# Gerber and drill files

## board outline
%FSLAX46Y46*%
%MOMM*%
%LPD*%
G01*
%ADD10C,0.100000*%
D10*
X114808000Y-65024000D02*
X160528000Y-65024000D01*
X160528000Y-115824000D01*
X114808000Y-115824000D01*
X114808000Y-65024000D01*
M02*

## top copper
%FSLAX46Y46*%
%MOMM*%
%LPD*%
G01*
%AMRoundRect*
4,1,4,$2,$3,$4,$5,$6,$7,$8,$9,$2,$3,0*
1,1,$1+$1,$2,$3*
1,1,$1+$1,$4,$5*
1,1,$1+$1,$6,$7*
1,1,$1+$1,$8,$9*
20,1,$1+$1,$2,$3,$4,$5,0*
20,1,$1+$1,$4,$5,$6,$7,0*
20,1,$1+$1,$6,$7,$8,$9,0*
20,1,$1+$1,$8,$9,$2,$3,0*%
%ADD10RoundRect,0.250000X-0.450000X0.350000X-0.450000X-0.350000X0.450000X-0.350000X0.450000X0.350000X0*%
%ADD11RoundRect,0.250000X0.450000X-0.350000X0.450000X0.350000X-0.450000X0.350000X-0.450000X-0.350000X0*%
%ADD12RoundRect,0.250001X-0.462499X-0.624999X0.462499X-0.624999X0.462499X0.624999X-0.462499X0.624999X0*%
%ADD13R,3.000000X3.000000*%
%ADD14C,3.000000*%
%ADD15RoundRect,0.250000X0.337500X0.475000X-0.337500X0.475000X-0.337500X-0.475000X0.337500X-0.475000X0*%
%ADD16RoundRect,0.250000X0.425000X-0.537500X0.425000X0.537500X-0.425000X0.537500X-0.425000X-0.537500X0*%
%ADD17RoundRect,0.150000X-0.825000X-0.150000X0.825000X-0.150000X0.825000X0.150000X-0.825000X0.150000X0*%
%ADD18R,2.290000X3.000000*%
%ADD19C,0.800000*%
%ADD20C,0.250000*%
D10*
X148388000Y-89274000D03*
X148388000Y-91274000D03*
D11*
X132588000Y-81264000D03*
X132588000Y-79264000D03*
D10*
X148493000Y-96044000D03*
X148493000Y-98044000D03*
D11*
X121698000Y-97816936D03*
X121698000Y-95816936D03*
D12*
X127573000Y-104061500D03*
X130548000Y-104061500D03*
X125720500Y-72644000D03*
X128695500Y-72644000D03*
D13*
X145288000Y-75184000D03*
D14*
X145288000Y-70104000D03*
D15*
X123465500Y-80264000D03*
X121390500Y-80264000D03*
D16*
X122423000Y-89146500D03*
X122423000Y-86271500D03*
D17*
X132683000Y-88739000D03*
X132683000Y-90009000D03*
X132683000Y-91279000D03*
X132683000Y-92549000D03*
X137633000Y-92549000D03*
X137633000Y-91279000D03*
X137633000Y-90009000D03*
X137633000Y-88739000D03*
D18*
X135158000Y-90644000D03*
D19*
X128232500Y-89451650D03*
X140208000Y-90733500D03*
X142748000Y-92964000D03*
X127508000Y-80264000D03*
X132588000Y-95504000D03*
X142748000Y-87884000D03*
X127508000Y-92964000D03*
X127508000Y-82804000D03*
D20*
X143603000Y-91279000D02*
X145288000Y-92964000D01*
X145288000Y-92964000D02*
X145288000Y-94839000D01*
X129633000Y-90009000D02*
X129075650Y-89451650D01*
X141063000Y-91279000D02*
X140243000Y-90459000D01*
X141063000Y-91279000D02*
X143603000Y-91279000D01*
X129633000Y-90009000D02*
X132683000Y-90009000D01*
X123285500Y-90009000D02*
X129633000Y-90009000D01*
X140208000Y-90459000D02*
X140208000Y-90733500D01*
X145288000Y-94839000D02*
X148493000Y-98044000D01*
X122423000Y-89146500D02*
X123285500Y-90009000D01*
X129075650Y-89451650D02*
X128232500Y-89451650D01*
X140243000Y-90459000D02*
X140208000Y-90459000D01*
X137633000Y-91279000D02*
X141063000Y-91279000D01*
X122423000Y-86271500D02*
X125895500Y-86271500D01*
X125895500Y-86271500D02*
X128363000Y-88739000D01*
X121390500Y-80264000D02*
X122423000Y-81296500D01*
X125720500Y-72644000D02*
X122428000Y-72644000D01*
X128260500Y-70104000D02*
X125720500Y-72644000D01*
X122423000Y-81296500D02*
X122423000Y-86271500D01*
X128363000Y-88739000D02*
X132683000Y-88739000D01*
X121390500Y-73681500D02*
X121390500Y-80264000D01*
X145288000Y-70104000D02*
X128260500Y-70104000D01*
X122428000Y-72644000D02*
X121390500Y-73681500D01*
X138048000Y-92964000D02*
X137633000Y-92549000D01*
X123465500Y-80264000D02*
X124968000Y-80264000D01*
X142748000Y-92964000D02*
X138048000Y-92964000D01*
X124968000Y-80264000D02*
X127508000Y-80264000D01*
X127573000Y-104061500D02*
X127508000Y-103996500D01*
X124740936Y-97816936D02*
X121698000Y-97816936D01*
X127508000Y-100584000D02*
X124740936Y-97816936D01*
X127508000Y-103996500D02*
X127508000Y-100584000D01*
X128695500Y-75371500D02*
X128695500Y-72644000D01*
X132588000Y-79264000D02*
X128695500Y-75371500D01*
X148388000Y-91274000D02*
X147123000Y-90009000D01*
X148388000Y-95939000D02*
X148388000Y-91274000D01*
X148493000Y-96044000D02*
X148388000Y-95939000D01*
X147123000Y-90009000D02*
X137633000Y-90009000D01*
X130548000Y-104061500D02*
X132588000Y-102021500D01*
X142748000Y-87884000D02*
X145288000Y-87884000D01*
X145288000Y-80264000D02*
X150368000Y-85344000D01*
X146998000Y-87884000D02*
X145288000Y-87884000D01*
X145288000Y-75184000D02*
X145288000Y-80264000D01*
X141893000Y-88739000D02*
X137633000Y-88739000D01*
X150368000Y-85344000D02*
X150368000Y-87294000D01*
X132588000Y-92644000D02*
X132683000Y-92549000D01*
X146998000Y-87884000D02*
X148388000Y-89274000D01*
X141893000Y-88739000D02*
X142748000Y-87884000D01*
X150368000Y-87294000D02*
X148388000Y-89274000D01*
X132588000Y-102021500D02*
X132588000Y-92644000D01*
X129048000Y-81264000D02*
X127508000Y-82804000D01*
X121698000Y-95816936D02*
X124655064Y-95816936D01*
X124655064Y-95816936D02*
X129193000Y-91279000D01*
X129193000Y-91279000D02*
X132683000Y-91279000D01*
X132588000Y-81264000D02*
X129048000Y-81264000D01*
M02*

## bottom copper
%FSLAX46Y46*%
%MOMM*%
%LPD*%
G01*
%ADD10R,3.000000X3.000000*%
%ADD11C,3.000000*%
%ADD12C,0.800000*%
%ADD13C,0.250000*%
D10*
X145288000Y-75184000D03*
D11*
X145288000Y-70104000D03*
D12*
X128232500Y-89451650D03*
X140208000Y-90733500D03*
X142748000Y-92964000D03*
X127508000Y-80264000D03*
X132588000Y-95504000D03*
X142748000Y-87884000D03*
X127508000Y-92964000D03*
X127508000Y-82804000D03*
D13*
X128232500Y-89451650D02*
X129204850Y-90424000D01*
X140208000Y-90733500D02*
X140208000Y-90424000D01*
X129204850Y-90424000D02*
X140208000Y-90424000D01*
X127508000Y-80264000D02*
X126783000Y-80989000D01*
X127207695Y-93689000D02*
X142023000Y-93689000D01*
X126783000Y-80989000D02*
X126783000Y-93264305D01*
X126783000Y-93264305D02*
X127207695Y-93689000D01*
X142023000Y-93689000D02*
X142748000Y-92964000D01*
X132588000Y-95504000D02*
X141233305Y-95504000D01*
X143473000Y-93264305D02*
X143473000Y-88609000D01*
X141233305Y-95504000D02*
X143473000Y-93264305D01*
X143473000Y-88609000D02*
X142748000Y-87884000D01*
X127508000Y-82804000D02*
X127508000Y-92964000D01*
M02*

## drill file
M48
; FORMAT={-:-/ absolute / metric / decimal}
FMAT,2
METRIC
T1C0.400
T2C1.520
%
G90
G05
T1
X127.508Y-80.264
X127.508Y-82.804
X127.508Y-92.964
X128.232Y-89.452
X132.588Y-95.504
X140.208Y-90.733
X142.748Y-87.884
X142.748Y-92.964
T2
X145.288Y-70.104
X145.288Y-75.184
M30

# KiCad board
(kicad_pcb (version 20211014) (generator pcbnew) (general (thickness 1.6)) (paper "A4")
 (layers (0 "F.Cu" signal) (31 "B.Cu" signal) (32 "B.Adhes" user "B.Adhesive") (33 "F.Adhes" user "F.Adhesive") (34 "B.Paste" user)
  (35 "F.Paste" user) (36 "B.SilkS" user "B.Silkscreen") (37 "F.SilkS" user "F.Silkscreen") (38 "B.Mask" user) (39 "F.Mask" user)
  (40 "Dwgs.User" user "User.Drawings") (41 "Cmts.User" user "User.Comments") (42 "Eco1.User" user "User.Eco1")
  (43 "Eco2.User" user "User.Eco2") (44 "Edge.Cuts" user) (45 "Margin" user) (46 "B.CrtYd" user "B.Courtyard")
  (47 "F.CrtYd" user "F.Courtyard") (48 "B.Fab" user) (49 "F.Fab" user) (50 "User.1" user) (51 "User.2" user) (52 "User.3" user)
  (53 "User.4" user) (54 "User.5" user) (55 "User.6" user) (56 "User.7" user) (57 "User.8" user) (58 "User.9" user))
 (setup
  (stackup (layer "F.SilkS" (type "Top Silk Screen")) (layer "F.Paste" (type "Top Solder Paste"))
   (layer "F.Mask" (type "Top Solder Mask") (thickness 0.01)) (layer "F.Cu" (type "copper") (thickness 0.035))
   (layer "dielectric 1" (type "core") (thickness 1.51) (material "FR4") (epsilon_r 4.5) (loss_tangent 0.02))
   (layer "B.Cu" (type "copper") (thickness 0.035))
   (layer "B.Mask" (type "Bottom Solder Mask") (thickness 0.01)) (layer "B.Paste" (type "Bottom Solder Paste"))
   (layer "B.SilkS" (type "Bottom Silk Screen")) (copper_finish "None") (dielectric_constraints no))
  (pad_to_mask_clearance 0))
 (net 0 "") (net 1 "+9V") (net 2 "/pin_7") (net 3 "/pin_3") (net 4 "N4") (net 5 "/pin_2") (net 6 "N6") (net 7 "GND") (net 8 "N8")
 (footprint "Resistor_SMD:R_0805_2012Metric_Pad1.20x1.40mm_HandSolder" (layer "F.Cu") (at 148.388 90.274 -90)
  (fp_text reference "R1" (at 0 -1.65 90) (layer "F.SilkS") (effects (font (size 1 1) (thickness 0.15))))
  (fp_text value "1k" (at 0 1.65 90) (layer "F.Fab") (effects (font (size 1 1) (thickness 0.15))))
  (pad "1" smd roundrect (at -1 0 270) (size 1.2 1.4) (layers "F.Cu" "F.Paste" "F.Mask") (roundrect_rratio 0.208333) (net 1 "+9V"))
  (pad "2" smd roundrect (at 1 0 270) (size 1.2 1.4) (layers "F.Cu" "F.Paste" "F.Mask") (roundrect_rratio 0.208333) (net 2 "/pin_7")))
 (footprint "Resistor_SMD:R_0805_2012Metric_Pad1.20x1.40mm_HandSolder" (layer "F.Cu") (at 132.588 80.264 90)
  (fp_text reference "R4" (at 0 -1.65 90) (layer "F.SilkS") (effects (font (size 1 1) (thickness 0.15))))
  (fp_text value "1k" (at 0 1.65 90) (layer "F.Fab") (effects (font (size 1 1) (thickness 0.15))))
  (pad "1" smd roundrect (at -1 0 90) (size 1.2 1.4) (layers "F.Cu" "F.Paste" "F.Mask") (roundrect_rratio 0.208333) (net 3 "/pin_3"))
  (pad "2" smd roundrect (at 1 0 90) (size 1.2 1.4) (layers "F.Cu" "F.Paste" "F.Mask") (roundrect_rratio 0.208333) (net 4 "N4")))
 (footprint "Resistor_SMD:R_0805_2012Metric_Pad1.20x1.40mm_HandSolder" (layer "F.Cu") (at 148.493 97.044 -90)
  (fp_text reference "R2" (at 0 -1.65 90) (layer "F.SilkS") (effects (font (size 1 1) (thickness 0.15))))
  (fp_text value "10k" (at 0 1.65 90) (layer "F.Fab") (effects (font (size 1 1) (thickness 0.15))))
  (pad "1" smd roundrect (at -1 0 270) (size 1.2 1.4) (layers "F.Cu" "F.Paste" "F.Mask") (roundrect_rratio 0.208333) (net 2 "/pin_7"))
  (pad "2" smd roundrect (at 1 0 270) (size 1.2 1.4) (layers "F.Cu" "F.Paste" "F.Mask") (roundrect_rratio 0.208333) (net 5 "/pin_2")))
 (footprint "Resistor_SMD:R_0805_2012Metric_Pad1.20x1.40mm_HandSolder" (layer "F.Cu") (at 121.698 96.816936 90)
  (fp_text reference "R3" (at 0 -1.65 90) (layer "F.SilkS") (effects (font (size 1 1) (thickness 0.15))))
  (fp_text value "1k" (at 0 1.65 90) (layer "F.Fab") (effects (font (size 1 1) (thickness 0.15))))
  (pad "1" smd roundrect (at -1 0 90) (size 1.2 1.4) (layers "F.Cu" "F.Paste" "F.Mask") (roundrect_rratio 0.208333) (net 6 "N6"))
  (pad "2" smd roundrect (at 1 0 90) (size 1.2 1.4) (layers "F.Cu" "F.Paste" "F.Mask") (roundrect_rratio 0.208333) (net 3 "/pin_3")))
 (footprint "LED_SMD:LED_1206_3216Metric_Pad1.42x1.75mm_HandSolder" (layer "F.Cu") (at 129.0605 104.0615)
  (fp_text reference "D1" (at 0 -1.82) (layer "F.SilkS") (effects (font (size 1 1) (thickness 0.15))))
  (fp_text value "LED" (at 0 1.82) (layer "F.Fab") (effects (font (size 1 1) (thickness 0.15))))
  (pad "1" smd roundrect (at -1.4875 0) (size 1.425 1.75) (layers "F.Cu" "F.Paste" "F.Mask") (roundrect_rratio 0.175439) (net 6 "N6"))
  (pad "2" smd roundrect (at 1.4875 0) (size 1.425 1.75) (layers "F.Cu" "F.Paste" "F.Mask") (roundrect_rratio 0.175439) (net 1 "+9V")))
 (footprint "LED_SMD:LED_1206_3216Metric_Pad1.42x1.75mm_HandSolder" (layer "F.Cu") (at 127.208 72.644)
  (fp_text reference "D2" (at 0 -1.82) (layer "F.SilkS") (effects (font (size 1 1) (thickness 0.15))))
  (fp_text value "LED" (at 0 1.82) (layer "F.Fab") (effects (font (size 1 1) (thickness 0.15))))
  (pad "1" smd roundrect (at -1.4875 0) (size 1.425 1.75) (layers "F.Cu" "F.Paste" "F.Mask") (roundrect_rratio 0.175439) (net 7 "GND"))
  (pad "2" smd roundrect (at 1.4875 0) (size 1.425 1.75) (layers "F.Cu" "F.Paste" "F.Mask") (roundrect_rratio 0.175439) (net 4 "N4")))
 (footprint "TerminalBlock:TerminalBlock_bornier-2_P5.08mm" (layer "F.Cu") (at 145.288 75.184 90)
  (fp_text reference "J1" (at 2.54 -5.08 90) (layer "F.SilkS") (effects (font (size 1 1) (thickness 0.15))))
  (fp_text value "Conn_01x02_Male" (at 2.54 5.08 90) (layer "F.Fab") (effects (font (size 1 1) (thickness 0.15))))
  (pad "1" thru_hole rect (at 0 0 90) (size 3 3) (drill 1.52) (layers F&B.Cu *.Mask) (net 1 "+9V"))
  (pad "2" thru_hole circle (at 5.08 0 90) (size 3 3) (drill 1.52) (layers F&B.Cu *.Mask) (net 7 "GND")))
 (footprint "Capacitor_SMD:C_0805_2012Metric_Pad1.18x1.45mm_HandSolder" (layer "F.Cu") (at 122.428 80.264 180)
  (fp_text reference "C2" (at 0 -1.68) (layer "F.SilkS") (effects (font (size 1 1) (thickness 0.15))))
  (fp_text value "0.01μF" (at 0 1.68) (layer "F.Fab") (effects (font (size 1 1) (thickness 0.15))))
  (pad "1" smd roundrect (at -1.0375 0 180) (size 1.175 1.45) (layers "F.Cu" "F.Paste" "F.Mask") (roundrect_rratio 0.212766) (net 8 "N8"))
  (pad "2" smd roundrect (at 1.0375 0 180) (size 1.175 1.45) (layers "F.Cu" "F.Paste" "F.Mask") (roundrect_rratio 0.212766) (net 7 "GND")))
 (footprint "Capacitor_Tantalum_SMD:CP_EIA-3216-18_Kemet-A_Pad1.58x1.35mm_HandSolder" (layer "F.Cu") (at 122.423 87.709 90)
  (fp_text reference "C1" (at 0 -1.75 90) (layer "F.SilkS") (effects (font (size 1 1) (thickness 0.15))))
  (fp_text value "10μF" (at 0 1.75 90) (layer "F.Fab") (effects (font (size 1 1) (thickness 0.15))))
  (pad "1" smd roundrect (at -1.4375 0 90) (size 1.575 1.35) (layers "F.Cu" "F.Paste" "F.Mask") (roundrect_rratio 0.185185) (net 5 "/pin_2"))
  (pad "2" smd roundrect (at 1.4375 0 90) (size 1.575 1.35) (layers "F.Cu" "F.Paste" "F.Mask") (roundrect_rratio 0.185185) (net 7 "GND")))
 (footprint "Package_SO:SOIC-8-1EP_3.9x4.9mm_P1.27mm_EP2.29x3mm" (layer "F.Cu") (at 135.158 90.644)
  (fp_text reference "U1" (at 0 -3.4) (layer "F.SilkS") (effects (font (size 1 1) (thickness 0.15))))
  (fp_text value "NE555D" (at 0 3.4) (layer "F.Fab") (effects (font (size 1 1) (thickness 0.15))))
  (pad "" smd roundrect (at -0.57 -0.75) (size 0.92 1.21) (layers "F.Paste") (roundrect_rratio 0.25))
  (pad "" smd roundrect (at 0.57 0.75) (size 0.92 1.21) (layers "F.Paste") (roundrect_rratio 0.25))
  (pad "" smd roundrect (at -0.57 0.75) (size 0.92 1.21) (layers "F.Paste") (roundrect_rratio 0.25))
  (pad "" smd roundrect (at 0.57 -0.75) (size 0.92 1.21) (layers "F.Paste") (roundrect_rratio 0.25))
  (pad "1" smd roundrect (at -2.475 -1.905) (size 1.95 0.6) (layers "F.Cu" "F.Paste" "F.Mask") (roundrect_rratio 0.25) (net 7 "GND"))
  (pad "2" smd roundrect (at -2.475 -0.635) (size 1.95 0.6) (layers "F.Cu" "F.Paste" "F.Mask") (roundrect_rratio 0.25) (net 5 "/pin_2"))
  (pad "3" smd roundrect (at -2.475 0.635) (size 1.95 0.6) (layers "F.Cu" "F.Paste" "F.Mask") (roundrect_rratio 0.25) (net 3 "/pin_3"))
  (pad "4" smd roundrect (at -2.475 1.905) (size 1.95 0.6) (layers "F.Cu" "F.Paste" "F.Mask") (roundrect_rratio 0.25) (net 1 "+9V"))
  (pad "5" smd roundrect (at 2.475 1.905) (size 1.95 0.6) (layers "F.Cu" "F.Paste" "F.Mask") (roundrect_rratio 0.25) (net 8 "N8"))
  (pad "6" smd roundrect (at 2.475 0.635) (size 1.95 0.6) (layers "F.Cu" "F.Paste" "F.Mask") (roundrect_rratio 0.25) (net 5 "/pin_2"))
  (pad "7" smd roundrect (at 2.475 -0.635) (size 1.95 0.6) (layers "F.Cu" "F.Paste" "F.Mask") (roundrect_rratio 0.25) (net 2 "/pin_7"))
  (pad "8" smd roundrect (at 2.475 -1.905) (size 1.95 0.6) (layers "F.Cu" "F.Paste" "F.Mask") (roundrect_rratio 0.25) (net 1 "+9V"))
  (pad "9" smd rect (at 0 0) (size 2.29 3) (layers "F.Cu" "F.Mask")))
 (gr_rect (start 114.808 65.024) (end 160.528 115.824) (layer "Edge.Cuts") (width 0.1) (fill none))
 (segment (start 143.603 91.279) (end 145.288 92.964) (width 0.25) (layer "F.Cu") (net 5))
 (segment (start 145.288 92.964) (end 145.288 94.839) (width 0.25) (layer "F.Cu") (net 5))
 (segment (start 129.633 90.009) (end 129.07565 89.45165) (width 0.25) (layer "F.Cu") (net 5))
 (segment (start 141.063 91.279) (end 140.243 90.459) (width 0.25) (layer "F.Cu") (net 5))
 (segment (start 141.063 91.279) (end 143.603 91.279) (width 0.25) (layer "F.Cu") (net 5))
 (segment (start 129.633 90.009) (end 132.683 90.009) (width 0.25) (layer "F.Cu") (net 5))
 (segment (start 123.2855 90.009) (end 129.633 90.009) (width 0.25) (layer "F.Cu") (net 5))
 (segment (start 140.208 90.459) (end 140.208 90.7335) (width 0.25) (layer "F.Cu") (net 5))
 (segment (start 145.288 94.839) (end 148.493 98.044) (width 0.25) (layer "F.Cu") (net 5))
 (segment (start 122.423 89.1465) (end 123.2855 90.009) (width 0.25) (layer "F.Cu") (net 5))
 (segment (start 129.07565 89.45165) (end 128.2325 89.45165) (width 0.25) (layer "F.Cu") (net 5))
 (segment (start 140.243 90.459) (end 140.208 90.459) (width 0.25) (layer "F.Cu") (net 5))
 (segment (start 137.633 91.279) (end 141.063 91.279) (width 0.25) (layer "F.Cu") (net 5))
 (via (at 128.2325 89.45165) (size 0.8) (drill 0.4) (layers "F.Cu" "B.Cu") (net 5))
 (via (at 140.208 90.7335) (size 0.8) (drill 0.4) (layers "F.Cu" "B.Cu") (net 5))
 (segment (start 128.2325 89.45165) (end 129.20485 90.424) (width 0.25) (layer "B.Cu") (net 5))
 (segment (start 140.208 90.7335) (end 140.208 90.424) (width 0.25) (layer "B.Cu") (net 5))
 (segment (start 129.20485 90.424) (end 140.208 90.424) (width 0.25) (layer "B.Cu") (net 5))
 (segment (start 122.423 86.2715) (end 125.8955 86.2715) (width 0.25) (layer "F.Cu") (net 7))
 (segment (start 125.8955 86.2715) (end 128.363 88.739) (width 0.25) (layer "F.Cu") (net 7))
 (segment (start 121.3905 80.264) (end 122.423 81.2965) (width 0.25) (layer "F.Cu") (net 7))
 (segment (start 125.7205 72.644) (end 122.428 72.644) (width 0.25) (layer "F.Cu") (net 7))
 (segment (start 128.2605 70.104) (end 125.7205 72.644) (width 0.25) (layer "F.Cu") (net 7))
 (segment (start 122.423 81.2965) (end 122.423 86.2715) (width 0.25) (layer "F.Cu") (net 7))
 (segment (start 128.363 88.739) (end 132.683 88.739) (width 0.25) (layer "F.Cu") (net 7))
 (segment (start 121.3905 73.6815) (end 121.3905 80.264) (width 0.25) (layer "F.Cu") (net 7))
 (segment (start 145.288 70.104) (end 128.2605 70.104) (width 0.25) (layer "F.Cu") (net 7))
 (segment (start 122.428 72.644) (end 121.3905 73.6815) (width 0.25) (layer "F.Cu") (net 7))
 (segment (start 138.048 92.964) (end 137.633 92.549) (width 0.25) (layer "F.Cu") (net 8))
 (segment (start 123.4655 80.264) (end 124.968 80.264) (width 0.25) (layer "F.Cu") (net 8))
 (segment (start 142.748 92.964) (end 138.048 92.964) (width 0.25) (layer "F.Cu") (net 8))
 (segment (start 124.968 80.264) (end 127.508 80.264) (width 0.25) (layer "F.Cu") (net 8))
 (via (at 142.748 92.964) (size 0.8) (drill 0.4) (layers "F.Cu" "B.Cu") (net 8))
 (via (at 127.508 80.264) (size 0.8) (drill 0.4) (layers "F.Cu" "B.Cu") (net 8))
 (segment (start 127.508 80.264) (end 126.783 80.989) (width 0.25) (layer "B.Cu") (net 8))
 (segment (start 127.207695 93.689) (end 142.023 93.689) (width 0.25) (layer "B.Cu") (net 8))
 (segment (start 126.783 80.989) (end 126.783 93.264305) (width 0.25) (layer "B.Cu") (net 8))
 (segment (start 126.783 93.264305) (end 127.207695 93.689) (width 0.25) (layer "B.Cu") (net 8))
 (segment (start 142.023 93.689) (end 142.748 92.964) (width 0.25) (layer "B.Cu") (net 8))
 (segment (start 127.573 104.0615) (end 127.508 103.9965) (width 0.25) (layer "F.Cu") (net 6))
 (segment (start 124.740936 97.816936) (end 121.698 97.816936) (width 0.25) (layer "F.Cu") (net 6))
 (segment (start 127.508 100.584) (end 124.740936 97.816936) (width 0.25) (layer "F.Cu") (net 6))
 (segment (start 127.508 103.9965) (end 127.508 100.584) (width 0.25) (layer "F.Cu") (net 6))
 (segment (start 128.6955 75.3715) (end 128.6955 72.644) (width 0.25) (layer "F.Cu") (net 4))
 (segment (start 132.588 79.264) (end 128.6955 75.3715) (width 0.25) (layer "F.Cu") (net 4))
 (segment (start 148.388 91.274) (end 147.123 90.009) (width 0.25) (layer "F.Cu") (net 2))
 (segment (start 148.388 95.939) (end 148.388 91.274) (width 0.25) (layer "F.Cu") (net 2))
 (segment (start 148.493 96.044) (end 148.388 95.939) (width 0.25) (layer "F.Cu") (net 2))
 (segment (start 147.123 90.009) (end 137.633 90.009) (width 0.25) (layer "F.Cu") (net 2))
 (segment (start 130.548 104.0615) (end 132.588 102.0215) (width 0.25) (layer "F.Cu") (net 1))
 (segment (start 142.748 87.884) (end 145.288 87.884) (width 0.25) (layer "F.Cu") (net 1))
 (segment (start 145.288 80.264) (end 150.368 85.344) (width 0.25) (layer "F.Cu") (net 1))
 (segment (start 146.998 87.884) (end 145.288 87.884) (width 0.25) (layer "F.Cu") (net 1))
 (segment (start 145.288 75.184) (end 145.288 80.264) (width 0.25) (layer "F.Cu") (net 1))
 (segment (start 141.893 88.739) (end 137.633 88.739) (width 0.25) (layer "F.Cu") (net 1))
 (segment (start 150.368 85.344) (end 150.368 87.294) (width 0.25) (layer "F.Cu") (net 1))
 (segment (start 132.588 92.644) (end 132.683 92.549) (width 0.25) (layer "F.Cu") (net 1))
 (segment (start 146.998 87.884) (end 148.388 89.274) (width 0.25) (layer "F.Cu") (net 1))
 (segment (start 141.893 88.739) (end 142.748 87.884) (width 0.25) (layer "F.Cu") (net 1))
 (segment (start 150.368 87.294) (end 148.388 89.274) (width 0.25) (layer "F.Cu") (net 1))
 (segment (start 132.588 102.0215) (end 132.588 92.644) (width 0.25) (layer "F.Cu") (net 1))
 (via (at 132.588 95.504) (size 0.8) (drill 0.4) (layers "F.Cu" "B.Cu") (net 1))
 (via (at 142.748 87.884) (size 0.8) (drill 0.4) (layers "F.Cu" "B.Cu") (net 1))
 (segment (start 132.588 95.504) (end 141.233305 95.504) (width 0.25) (layer "B.Cu") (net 1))
 (segment (start 143.473 93.264305) (end 143.473 88.609) (width 0.25) (layer "B.Cu") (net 1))
 (segment (start 141.233305 95.504) (end 143.473 93.264305) (width 0.25) (layer "B.Cu") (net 1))
 (segment (start 143.473 88.609) (end 142.748 87.884) (width 0.25) (layer "B.Cu") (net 1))
 (segment (start 129.048 81.264) (end 127.508 82.804) (width 0.25) (layer "F.Cu") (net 3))
 (segment (start 121.698 95.816936) (end 124.655064 95.816936) (width 0.25) (layer "F.Cu") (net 3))
 (segment (start 124.655064 95.816936) (end 129.193 91.279) (width 0.25) (layer "F.Cu") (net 3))
 (segment (start 129.193 91.279) (end 132.683 91.279) (width 0.25) (layer "F.Cu") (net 3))
 (segment (start 132.588 81.264) (end 129.048 81.264) (width 0.25) (layer "F.Cu") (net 3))
 (via (at 127.508 92.964) (size 0.8) (drill 0.4) (layers "F.Cu" "B.Cu") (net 3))
 (via (at 127.508 82.804) (size 0.8) (drill 0.4) (layers "F.Cu" "B.Cu") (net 3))
 (segment (start 127.508 82.804) (end 127.508 92.964) (width 0.25) (layer "B.Cu") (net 3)))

